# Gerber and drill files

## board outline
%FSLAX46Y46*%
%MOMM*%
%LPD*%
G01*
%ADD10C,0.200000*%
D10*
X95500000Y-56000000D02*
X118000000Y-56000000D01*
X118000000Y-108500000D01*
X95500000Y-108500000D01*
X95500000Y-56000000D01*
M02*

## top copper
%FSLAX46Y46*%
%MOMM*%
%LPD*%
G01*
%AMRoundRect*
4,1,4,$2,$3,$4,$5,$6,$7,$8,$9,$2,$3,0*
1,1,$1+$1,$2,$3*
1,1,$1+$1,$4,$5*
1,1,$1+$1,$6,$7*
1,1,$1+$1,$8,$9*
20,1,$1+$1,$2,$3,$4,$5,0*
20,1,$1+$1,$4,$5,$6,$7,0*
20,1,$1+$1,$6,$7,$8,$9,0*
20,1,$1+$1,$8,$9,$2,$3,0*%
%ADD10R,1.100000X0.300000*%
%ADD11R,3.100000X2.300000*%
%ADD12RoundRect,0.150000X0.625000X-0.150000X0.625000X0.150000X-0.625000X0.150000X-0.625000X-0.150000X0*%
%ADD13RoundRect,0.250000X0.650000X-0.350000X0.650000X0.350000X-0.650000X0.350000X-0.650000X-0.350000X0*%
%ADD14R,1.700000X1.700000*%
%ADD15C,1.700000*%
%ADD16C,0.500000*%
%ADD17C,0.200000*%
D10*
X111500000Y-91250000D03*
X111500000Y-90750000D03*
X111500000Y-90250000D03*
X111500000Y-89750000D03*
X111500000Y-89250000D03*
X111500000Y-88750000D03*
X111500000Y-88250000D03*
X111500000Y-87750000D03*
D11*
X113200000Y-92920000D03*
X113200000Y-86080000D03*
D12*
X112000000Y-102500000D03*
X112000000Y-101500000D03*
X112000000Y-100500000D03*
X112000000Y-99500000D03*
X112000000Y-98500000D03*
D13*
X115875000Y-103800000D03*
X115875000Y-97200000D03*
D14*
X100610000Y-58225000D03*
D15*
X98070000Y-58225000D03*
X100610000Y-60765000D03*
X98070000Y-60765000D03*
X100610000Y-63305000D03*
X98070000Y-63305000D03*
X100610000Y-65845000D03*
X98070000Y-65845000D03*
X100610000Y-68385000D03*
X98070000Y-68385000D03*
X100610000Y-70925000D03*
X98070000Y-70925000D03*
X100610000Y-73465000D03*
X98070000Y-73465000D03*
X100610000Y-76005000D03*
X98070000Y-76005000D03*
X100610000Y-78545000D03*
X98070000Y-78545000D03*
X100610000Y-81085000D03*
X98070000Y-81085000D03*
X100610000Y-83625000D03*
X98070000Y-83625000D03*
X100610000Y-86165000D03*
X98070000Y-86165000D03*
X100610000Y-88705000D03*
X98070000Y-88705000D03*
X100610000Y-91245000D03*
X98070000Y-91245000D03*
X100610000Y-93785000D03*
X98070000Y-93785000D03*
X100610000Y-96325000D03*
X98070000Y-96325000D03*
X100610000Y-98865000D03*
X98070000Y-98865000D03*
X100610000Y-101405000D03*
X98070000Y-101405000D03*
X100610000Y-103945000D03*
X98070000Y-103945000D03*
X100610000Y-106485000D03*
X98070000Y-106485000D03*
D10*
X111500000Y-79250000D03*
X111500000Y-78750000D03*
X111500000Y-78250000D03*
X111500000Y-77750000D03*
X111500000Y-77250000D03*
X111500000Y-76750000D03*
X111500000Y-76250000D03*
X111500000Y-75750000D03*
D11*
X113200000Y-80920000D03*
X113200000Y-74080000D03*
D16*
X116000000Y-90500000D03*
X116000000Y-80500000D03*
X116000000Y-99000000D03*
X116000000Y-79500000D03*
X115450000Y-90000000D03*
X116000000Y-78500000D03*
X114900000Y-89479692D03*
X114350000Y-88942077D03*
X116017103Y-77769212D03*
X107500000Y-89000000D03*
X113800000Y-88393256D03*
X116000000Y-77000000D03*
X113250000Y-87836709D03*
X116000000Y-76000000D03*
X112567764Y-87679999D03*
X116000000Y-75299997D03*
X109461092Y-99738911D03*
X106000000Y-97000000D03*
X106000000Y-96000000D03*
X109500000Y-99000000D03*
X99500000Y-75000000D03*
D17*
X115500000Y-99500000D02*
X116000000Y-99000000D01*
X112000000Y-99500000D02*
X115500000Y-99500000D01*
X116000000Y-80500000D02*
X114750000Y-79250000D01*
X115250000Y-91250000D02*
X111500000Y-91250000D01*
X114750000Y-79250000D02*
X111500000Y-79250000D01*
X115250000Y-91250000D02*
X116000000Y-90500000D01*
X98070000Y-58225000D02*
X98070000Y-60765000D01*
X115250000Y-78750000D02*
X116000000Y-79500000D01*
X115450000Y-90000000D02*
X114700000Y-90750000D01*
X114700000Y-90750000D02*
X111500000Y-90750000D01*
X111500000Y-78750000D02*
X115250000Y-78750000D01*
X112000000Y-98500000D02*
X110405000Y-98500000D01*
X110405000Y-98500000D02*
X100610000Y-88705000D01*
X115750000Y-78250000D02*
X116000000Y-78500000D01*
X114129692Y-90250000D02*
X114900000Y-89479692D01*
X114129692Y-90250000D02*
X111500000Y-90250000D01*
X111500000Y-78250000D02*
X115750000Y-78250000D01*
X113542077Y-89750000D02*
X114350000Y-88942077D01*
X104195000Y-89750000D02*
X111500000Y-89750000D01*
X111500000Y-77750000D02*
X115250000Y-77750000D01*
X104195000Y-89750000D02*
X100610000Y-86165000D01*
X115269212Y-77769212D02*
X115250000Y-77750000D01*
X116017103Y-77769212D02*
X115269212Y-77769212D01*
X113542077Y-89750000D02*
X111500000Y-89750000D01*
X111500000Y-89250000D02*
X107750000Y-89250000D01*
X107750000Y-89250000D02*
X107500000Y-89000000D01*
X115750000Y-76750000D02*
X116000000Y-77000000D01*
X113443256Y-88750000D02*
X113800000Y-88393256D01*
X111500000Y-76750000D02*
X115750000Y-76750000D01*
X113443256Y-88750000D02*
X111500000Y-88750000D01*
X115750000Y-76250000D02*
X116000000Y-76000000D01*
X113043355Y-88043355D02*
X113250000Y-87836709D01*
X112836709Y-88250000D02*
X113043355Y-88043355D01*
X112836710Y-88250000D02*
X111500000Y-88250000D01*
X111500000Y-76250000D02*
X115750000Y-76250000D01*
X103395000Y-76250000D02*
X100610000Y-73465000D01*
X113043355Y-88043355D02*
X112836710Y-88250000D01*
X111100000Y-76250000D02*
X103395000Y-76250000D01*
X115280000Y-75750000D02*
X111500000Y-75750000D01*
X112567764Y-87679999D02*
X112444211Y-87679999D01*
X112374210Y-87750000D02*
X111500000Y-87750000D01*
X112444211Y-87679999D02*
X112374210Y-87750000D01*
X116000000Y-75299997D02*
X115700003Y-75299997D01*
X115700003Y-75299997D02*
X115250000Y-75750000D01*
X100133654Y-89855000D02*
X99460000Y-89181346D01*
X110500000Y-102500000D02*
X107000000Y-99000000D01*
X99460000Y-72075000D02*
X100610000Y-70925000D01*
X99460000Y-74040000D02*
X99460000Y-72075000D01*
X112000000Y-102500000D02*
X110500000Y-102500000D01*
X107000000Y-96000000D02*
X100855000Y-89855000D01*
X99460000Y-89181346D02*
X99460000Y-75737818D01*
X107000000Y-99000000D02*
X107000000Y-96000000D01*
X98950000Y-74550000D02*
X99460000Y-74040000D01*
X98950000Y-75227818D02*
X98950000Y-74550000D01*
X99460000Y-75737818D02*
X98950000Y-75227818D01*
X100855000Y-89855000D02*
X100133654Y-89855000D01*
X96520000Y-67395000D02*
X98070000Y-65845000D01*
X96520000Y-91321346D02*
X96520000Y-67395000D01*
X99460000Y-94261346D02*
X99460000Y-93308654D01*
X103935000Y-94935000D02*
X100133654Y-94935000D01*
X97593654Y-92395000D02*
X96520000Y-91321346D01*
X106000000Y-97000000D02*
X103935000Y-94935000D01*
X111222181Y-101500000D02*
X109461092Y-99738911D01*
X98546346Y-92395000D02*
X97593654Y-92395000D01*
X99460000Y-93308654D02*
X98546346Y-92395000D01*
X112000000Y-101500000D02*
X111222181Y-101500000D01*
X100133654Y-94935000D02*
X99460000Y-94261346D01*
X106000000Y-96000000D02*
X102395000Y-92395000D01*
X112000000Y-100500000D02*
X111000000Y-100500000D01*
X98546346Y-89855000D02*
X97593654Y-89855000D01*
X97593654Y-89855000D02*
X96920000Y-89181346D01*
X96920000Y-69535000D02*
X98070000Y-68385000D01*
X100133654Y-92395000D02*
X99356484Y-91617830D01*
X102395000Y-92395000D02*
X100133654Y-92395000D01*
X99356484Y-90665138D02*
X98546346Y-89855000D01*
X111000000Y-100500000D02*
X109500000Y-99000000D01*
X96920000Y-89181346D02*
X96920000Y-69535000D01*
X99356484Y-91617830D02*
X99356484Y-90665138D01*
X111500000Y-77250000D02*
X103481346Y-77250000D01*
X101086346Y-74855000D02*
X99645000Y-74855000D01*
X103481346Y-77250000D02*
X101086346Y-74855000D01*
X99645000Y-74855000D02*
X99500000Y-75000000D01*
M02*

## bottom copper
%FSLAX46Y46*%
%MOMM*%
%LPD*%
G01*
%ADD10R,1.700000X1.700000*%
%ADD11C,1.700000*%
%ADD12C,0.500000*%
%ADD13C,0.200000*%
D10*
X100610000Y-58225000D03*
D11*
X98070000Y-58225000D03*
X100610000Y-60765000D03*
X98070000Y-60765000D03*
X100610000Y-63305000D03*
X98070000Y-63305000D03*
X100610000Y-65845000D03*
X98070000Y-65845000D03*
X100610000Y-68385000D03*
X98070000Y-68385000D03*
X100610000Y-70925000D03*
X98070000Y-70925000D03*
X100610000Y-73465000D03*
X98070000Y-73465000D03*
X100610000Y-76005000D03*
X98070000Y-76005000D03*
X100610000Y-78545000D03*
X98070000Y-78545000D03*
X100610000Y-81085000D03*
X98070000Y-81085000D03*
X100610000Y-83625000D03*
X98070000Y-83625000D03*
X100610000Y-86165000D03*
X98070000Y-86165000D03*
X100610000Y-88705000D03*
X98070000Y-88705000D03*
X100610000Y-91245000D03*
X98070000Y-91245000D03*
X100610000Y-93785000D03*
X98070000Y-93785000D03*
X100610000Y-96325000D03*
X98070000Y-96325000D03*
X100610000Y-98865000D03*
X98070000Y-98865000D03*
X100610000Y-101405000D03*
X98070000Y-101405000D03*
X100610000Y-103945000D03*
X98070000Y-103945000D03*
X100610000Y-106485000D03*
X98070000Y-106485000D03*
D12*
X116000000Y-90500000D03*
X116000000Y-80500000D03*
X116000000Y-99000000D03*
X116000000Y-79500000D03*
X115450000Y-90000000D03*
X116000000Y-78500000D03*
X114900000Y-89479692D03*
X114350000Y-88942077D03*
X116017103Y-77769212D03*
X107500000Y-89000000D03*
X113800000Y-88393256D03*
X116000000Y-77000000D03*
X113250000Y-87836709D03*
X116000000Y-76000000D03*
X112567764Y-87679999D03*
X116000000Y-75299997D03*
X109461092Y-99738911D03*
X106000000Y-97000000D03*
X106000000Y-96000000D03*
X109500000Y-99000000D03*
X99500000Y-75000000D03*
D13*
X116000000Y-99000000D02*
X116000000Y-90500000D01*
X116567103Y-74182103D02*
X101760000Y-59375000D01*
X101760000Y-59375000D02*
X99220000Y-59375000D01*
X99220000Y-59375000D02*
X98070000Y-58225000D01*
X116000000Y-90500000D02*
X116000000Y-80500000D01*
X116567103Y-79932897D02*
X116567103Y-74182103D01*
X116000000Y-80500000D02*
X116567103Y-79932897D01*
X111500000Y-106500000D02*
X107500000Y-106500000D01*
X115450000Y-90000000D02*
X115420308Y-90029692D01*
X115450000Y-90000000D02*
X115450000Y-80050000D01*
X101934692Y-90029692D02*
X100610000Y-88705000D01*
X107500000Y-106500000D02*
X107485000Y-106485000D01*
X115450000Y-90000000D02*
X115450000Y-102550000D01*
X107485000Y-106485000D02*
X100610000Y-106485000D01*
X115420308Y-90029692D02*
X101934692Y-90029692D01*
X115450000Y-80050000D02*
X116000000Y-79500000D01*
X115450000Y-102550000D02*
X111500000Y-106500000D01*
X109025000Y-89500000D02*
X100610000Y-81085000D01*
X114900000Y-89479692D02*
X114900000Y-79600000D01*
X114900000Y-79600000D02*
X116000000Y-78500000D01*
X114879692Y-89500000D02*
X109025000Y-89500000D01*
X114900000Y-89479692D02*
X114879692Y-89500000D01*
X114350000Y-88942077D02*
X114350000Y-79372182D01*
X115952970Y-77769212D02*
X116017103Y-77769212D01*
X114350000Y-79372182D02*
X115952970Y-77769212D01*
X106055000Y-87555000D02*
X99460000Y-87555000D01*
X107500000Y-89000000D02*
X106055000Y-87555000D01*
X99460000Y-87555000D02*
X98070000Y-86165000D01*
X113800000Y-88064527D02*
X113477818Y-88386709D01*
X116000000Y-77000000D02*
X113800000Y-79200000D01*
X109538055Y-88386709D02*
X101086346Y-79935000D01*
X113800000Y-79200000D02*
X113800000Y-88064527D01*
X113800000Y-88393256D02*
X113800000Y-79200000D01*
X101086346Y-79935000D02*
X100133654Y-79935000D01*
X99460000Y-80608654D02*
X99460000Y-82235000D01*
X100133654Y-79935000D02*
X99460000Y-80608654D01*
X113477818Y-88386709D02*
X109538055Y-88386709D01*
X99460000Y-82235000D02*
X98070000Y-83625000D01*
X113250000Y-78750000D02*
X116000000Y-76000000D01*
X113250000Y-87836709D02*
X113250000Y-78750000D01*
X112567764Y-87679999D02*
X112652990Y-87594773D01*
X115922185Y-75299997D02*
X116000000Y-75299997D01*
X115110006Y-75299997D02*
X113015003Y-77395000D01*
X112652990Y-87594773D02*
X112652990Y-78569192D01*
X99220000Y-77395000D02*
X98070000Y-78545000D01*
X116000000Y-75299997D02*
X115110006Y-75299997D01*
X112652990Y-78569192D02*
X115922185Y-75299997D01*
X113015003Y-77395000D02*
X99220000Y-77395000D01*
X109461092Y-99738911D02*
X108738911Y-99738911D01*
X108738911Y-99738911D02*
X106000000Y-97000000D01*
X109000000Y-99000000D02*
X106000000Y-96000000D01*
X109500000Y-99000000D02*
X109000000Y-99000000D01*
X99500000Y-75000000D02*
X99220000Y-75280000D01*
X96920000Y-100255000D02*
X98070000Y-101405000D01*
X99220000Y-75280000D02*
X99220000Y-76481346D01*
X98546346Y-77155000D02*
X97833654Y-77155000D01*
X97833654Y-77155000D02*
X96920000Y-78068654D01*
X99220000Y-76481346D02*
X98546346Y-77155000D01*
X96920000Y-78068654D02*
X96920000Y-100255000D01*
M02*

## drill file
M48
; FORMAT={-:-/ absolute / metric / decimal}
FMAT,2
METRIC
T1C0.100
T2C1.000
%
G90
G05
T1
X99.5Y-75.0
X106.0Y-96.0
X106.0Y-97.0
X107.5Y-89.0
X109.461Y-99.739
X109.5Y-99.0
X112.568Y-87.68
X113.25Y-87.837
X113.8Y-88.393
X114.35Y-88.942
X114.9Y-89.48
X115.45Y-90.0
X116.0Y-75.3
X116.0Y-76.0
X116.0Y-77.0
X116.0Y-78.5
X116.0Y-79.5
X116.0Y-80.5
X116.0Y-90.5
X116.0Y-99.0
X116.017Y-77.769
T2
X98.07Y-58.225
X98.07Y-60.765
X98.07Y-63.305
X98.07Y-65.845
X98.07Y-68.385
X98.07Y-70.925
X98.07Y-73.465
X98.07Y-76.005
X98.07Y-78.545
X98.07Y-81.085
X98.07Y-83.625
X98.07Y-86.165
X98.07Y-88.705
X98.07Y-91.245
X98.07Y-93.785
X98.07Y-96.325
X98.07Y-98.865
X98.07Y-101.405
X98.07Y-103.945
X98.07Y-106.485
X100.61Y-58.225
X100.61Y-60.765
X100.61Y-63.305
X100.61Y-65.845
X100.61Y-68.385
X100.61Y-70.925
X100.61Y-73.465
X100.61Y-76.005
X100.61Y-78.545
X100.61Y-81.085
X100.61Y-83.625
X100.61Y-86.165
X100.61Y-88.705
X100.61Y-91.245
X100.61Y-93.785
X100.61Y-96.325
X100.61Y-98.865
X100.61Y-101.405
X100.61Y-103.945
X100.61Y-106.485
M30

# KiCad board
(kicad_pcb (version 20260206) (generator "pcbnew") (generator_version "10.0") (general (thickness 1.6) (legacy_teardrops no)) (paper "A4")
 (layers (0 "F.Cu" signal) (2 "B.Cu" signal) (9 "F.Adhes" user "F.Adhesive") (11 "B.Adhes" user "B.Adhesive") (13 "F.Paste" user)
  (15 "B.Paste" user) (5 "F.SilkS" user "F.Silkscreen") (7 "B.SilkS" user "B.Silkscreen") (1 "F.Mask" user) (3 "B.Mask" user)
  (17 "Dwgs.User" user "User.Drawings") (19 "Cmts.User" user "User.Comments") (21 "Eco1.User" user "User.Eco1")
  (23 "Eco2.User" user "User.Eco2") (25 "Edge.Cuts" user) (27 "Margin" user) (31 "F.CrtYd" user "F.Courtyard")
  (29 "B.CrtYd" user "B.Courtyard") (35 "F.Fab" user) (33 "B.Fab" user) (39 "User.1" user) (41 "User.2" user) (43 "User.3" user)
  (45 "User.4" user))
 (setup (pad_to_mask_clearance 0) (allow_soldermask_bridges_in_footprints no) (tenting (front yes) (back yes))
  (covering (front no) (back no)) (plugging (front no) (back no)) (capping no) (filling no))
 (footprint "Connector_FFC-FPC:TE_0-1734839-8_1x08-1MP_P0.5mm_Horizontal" (layer "F.Cu") (at 112.85 89.5 90)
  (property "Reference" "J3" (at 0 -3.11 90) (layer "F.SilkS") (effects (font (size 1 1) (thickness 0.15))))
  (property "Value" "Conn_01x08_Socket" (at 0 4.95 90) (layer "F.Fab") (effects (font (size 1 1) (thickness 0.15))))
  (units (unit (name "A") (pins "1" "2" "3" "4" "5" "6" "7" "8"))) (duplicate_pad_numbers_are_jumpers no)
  (pad "1" smd rect (at -1.75 -1.35 90) (size 0.3 1.1) (layers "F.Cu" "F.Mask" "F.Paste") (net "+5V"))
  (pad "2" smd rect (at -1.25 -1.35 90) (size 0.3 1.1) (layers "F.Cu" "F.Mask" "F.Paste") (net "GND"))
  (pad "3" smd rect (at -0.75 -1.35 90) (size 0.3 1.1) (layers "F.Cu" "F.Mask" "F.Paste") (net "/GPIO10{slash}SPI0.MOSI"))
  (pad "4" smd rect (at -0.25 -1.35 90) (size 0.3 1.1) (layers "F.Cu" "F.Mask" "F.Paste") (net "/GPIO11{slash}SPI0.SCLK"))
  (pad "5" smd rect (at 0.25 -1.35 90) (size 0.3 1.1) (layers "F.Cu" "F.Mask" "F.Paste") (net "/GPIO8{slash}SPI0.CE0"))
  (pad "6" smd rect (at 0.75 -1.35 90) (size 0.3 1.1) (layers "F.Cu" "F.Mask" "F.Paste") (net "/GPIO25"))
  (pad "7" smd rect (at 1.25 -1.35 90) (size 0.3 1.1) (layers "F.Cu" "F.Mask" "F.Paste") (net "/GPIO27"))
  (pad "8" smd rect (at 1.75 -1.35 90) (size 0.3 1.1) (layers "F.Cu" "F.Mask" "F.Paste") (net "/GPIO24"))
  (pad "MP" smd rect (at -3.42 0.35 90) (size 2.3 3.1) (layers "F.Cu" "F.Mask" "F.Paste"))
  (pad "MP" smd rect (at 3.42 0.35 90) (size 2.3 3.1) (layers "F.Cu" "F.Mask" "F.Paste")))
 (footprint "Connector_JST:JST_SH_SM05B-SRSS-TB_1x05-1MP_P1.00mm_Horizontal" (layer "F.Cu") (at 114 100.5 90)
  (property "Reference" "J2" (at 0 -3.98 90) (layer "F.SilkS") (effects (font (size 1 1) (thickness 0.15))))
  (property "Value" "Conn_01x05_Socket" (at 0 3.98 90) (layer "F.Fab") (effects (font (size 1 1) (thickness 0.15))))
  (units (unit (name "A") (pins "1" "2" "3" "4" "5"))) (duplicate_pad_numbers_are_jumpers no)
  (pad "1" smd roundrect (at -2 -2 90) (size 0.6 1.55) (layers "F.Cu" "F.Mask" "F.Paste") (roundrect_rratio 0.25) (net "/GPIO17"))
  (pad "2" smd roundrect (at -1 -2 90) (size 0.6 1.55) (layers "F.Cu" "F.Mask" "F.Paste") (roundrect_rratio 0.25) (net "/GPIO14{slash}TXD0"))
  (pad "3" smd roundrect (at 0 -2 90) (size 0.6 1.55) (layers "F.Cu" "F.Mask" "F.Paste") (roundrect_rratio 0.25) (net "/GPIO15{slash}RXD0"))
  (pad "4" smd roundrect (at 1 -2 90) (size 0.6 1.55) (layers "F.Cu" "F.Mask" "F.Paste") (roundrect_rratio 0.25) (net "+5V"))
  (pad "5" smd roundrect (at 2 -2 90) (size 0.6 1.55) (layers "F.Cu" "F.Mask" "F.Paste") (roundrect_rratio 0.25) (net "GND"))
  (pad "MP" smd roundrect (at -3.3 1.875 90) (size 1.2 1.8) (layers "F.Cu" "F.Mask" "F.Paste") (roundrect_rratio 0.208333))
  (pad "MP" smd roundrect (at 3.3 1.875 90) (size 1.2 1.8) (layers "F.Cu" "F.Mask" "F.Paste") (roundrect_rratio 0.208333)))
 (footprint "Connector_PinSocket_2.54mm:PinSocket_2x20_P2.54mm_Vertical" (layer "F.Cu") (at 100.61 58.225)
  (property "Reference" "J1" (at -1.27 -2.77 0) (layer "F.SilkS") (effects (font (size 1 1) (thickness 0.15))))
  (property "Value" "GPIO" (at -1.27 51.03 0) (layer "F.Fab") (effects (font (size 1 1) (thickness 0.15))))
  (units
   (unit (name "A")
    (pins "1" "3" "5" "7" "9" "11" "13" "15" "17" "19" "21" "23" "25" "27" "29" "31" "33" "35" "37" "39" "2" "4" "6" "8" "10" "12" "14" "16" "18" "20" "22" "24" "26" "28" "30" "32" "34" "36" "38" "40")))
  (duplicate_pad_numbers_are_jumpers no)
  (pad "1" thru_hole rect (at 0 0) (size 1.7 1.7) (drill 1) (layers "*.Cu" "*.Mask") (remove_unused_layers no) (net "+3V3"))
  (pad "2" thru_hole circle (at -2.54 0) (size 1.7 1.7) (drill 1) (layers "*.Cu" "*.Mask") (remove_unused_layers no) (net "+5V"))
  (pad "3" thru_hole circle (at 0 2.54) (size 1.7 1.7) (drill 1) (layers "*.Cu" "*.Mask") (remove_unused_layers no)
   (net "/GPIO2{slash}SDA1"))
  (pad "4" thru_hole circle (at -2.54 2.54) (size 1.7 1.7) (drill 1) (layers "*.Cu" "*.Mask") (remove_unused_layers no) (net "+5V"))
  (pad "5" thru_hole circle (at 0 5.08) (size 1.7 1.7) (drill 1) (layers "*.Cu" "*.Mask") (remove_unused_layers no)
   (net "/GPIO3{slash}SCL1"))
  (pad "6" thru_hole circle (at -2.54 5.08) (size 1.7 1.7) (drill 1) (layers "*.Cu" "*.Mask") (remove_unused_layers no) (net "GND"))
  (pad "7" thru_hole circle (at 0 7.62) (size 1.7 1.7) (drill 1) (layers "*.Cu" "*.Mask") (remove_unused_layers no)
   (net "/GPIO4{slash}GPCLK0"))
  (pad "8" thru_hole circle (at -2.54 7.62) (size 1.7 1.7) (drill 1) (layers "*.Cu" "*.Mask") (remove_unused_layers no)
   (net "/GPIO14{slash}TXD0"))
  (pad "9" thru_hole circle (at 0 10.16) (size 1.7 1.7) (drill 1) (layers "*.Cu" "*.Mask") (remove_unused_layers no) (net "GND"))
  (pad "10" thru_hole circle (at -2.54 10.16) (size 1.7 1.7) (drill 1) (layers "*.Cu" "*.Mask") (remove_unused_layers no)
   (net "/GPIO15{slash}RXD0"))
  (pad "11" thru_hole circle (at 0 12.7) (size 1.7 1.7) (drill 1) (layers "*.Cu" "*.Mask") (remove_unused_layers no) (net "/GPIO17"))
  (pad "12" thru_hole circle (at -2.54 12.7) (size 1.7 1.7) (drill 1) (layers "*.Cu" "*.Mask") (remove_unused_layers no)
   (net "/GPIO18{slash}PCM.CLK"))
  (pad "13" thru_hole circle (at 0 15.24) (size 1.7 1.7) (drill 1) (layers "*.Cu" "*.Mask") (remove_unused_layers no) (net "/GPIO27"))
  (pad "14" thru_hole circle (at -2.54 15.24) (size 1.7 1.7) (drill 1) (layers "*.Cu" "*.Mask") (remove_unused_layers no) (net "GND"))
  (pad "15" thru_hole circle (at 0 17.78) (size 1.7 1.7) (drill 1) (layers "*.Cu" "*.Mask") (remove_unused_layers no) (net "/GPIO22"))
  (pad "16" thru_hole circle (at -2.54 17.78) (size 1.7 1.7) (drill 1) (layers "*.Cu" "*.Mask") (remove_unused_layers no) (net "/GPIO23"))
  (pad "17" thru_hole circle (at 0 20.32) (size 1.7 1.7) (drill 1) (layers "*.Cu" "*.Mask") (remove_unused_layers no) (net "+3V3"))
  (pad "18" thru_hole circle (at -2.54 20.32) (size 1.7 1.7) (drill 1) (layers "*.Cu" "*.Mask") (remove_unused_layers no) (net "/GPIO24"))
  (pad "19" thru_hole circle (at 0 22.86) (size 1.7 1.7) (drill 1) (layers "*.Cu" "*.Mask") (remove_unused_layers no)
   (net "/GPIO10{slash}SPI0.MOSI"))
  (pad "20" thru_hole circle (at -2.54 22.86) (size 1.7 1.7) (drill 1) (layers "*.Cu" "*.Mask") (remove_unused_layers no) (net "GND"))
  (pad "21" thru_hole circle (at 0 25.4) (size 1.7 1.7) (drill 1) (layers "*.Cu" "*.Mask") (remove_unused_layers no)
   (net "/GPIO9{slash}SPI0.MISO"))
  (pad "22" thru_hole circle (at -2.54 25.4) (size 1.7 1.7) (drill 1) (layers "*.Cu" "*.Mask") (remove_unused_layers no) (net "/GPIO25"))
  (pad "23" thru_hole circle (at 0 27.94) (size 1.7 1.7) (drill 1) (layers "*.Cu" "*.Mask") (remove_unused_layers no)
   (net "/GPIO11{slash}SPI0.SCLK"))
  (pad "24" thru_hole circle (at -2.54 27.94) (size 1.7 1.7) (drill 1) (layers "*.Cu" "*.Mask") (remove_unused_layers no)
   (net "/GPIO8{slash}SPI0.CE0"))
  (pad "25" thru_hole circle (at 0 30.48) (size 1.7 1.7) (drill 1) (layers "*.Cu" "*.Mask") (remove_unused_layers no) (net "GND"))
  (pad "26" thru_hole circle (at -2.54 30.48) (size 1.7 1.7) (drill 1) (layers "*.Cu" "*.Mask") (remove_unused_layers no)
   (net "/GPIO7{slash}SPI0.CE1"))
  (pad "27" thru_hole circle (at 0 33.02) (size 1.7 1.7) (drill 1) (layers "*.Cu" "*.Mask") (remove_unused_layers no) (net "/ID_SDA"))
  (pad "28" thru_hole circle (at -2.54 33.02) (size 1.7 1.7) (drill 1) (layers "*.Cu" "*.Mask") (remove_unused_layers no) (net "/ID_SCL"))
  (pad "29" thru_hole circle (at 0 35.56) (size 1.7 1.7) (drill 1) (layers "*.Cu" "*.Mask") (remove_unused_layers no) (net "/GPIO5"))
  (pad "30" thru_hole circle (at -2.54 35.56) (size 1.7 1.7) (drill 1) (layers "*.Cu" "*.Mask") (remove_unused_layers no) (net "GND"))
  (pad "31" thru_hole circle (at 0 38.1) (size 1.7 1.7) (drill 1) (layers "*.Cu" "*.Mask") (remove_unused_layers no) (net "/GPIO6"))
  (pad "32" thru_hole circle (at -2.54 38.1) (size 1.7 1.7) (drill 1) (layers "*.Cu" "*.Mask") (remove_unused_layers no)
   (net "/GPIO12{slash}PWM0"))
  (pad "33" thru_hole circle (at 0 40.64) (size 1.7 1.7) (drill 1) (layers "*.Cu" "*.Mask") (remove_unused_layers no)
   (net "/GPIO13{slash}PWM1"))
  (pad "34" thru_hole circle (at -2.54 40.64) (size 1.7 1.7) (drill 1) (layers "*.Cu" "*.Mask") (remove_unused_layers no) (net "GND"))
  (pad "35" thru_hole circle (at 0 43.18) (size 1.7 1.7) (drill 1) (layers "*.Cu" "*.Mask") (remove_unused_layers no)
   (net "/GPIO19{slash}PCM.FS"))
  (pad "36" thru_hole circle (at -2.54 43.18) (size 1.7 1.7) (drill 1) (layers "*.Cu" "*.Mask") (remove_unused_layers no) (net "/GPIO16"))
  (pad "37" thru_hole circle (at 0 45.72) (size 1.7 1.7) (drill 1) (layers "*.Cu" "*.Mask") (remove_unused_layers no) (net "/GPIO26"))
  (pad "38" thru_hole circle (at -2.54 45.72) (size 1.7 1.7) (drill 1) (layers "*.Cu" "*.Mask") (remove_unused_layers no)
   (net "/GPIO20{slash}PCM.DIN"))
  (pad "39" thru_hole circle (at 0 48.26) (size 1.7 1.7) (drill 1) (layers "*.Cu" "*.Mask") (remove_unused_layers no) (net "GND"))
  (pad "40" thru_hole circle (at -2.54 48.26) (size 1.7 1.7) (drill 1) (layers "*.Cu" "*.Mask") (remove_unused_layers no)
   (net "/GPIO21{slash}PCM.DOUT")))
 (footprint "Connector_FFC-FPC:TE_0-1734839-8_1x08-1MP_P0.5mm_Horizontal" (layer "F.Cu") (at 112.85 77.5 90)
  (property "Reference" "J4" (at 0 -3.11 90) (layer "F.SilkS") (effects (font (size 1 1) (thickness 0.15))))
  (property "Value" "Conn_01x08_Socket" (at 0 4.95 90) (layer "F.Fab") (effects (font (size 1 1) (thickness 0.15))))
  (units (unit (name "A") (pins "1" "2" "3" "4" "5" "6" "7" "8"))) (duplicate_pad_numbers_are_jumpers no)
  (pad "1" smd rect (at -1.75 -1.35 90) (size 0.3 1.1) (layers "F.Cu" "F.Mask" "F.Paste") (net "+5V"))
  (pad "2" smd rect (at -1.25 -1.35 90) (size 0.3 1.1) (layers "F.Cu" "F.Mask" "F.Paste") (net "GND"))
  (pad "3" smd rect (at -0.75 -1.35 90) (size 0.3 1.1) (layers "F.Cu" "F.Mask" "F.Paste") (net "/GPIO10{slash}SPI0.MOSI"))
  (pad "4" smd rect (at -0.25 -1.35 90) (size 0.3 1.1) (layers "F.Cu" "F.Mask" "F.Paste") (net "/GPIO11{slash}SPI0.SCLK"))
  (pad "5" smd rect (at 0.25 -1.35 90) (size 0.3 1.1) (layers "F.Cu" "F.Mask" "F.Paste") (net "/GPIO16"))
  (pad "6" smd rect (at 0.75 -1.35 90) (size 0.3 1.1) (layers "F.Cu" "F.Mask" "F.Paste") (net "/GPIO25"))
  (pad "7" smd rect (at 1.25 -1.35 90) (size 0.3 1.1) (layers "F.Cu" "F.Mask" "F.Paste") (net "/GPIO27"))
  (pad "8" smd rect (at 1.75 -1.35 90) (size 0.3 1.1) (layers "F.Cu" "F.Mask" "F.Paste") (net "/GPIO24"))
  (pad "MP" smd rect (at -3.42 0.35 90) (size 2.3 3.1) (layers "F.Cu" "F.Mask" "F.Paste"))
  (pad "MP" smd rect (at 3.42 0.35 90) (size 2.3 3.1) (layers "F.Cu" "F.Mask" "F.Paste")))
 (gr_rect (start 95.5 56) (end 118 108.5) (stroke (width 0.2) (type solid)) (fill no) (layer "Edge.Cuts"))
 (segment (start 115.5 99.5) (end 116 99) (width 0.2) (layer "F.Cu") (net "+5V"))
 (segment (start 112 99.5) (end 115.5 99.5) (width 0.2) (layer "F.Cu") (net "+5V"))
 (segment (start 116 80.5) (end 114.75 79.25) (width 0.2) (layer "F.Cu") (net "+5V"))
 (segment (start 115.25 91.25) (end 111.5 91.25) (width 0.2) (layer "F.Cu") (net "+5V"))
 (segment (start 114.75 79.25) (end 111.5 79.25) (width 0.2) (layer "F.Cu") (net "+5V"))
 (segment (start 115.25 91.25) (end 116 90.5) (width 0.2) (layer "F.Cu") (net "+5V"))
 (segment (start 98.07 58.225) (end 98.07 60.765) (width 0.2) (layer "F.Cu") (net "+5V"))
 (via micro (at 116 90.5) (size 0.5) (drill 0.1) (layers "F.Cu" "B.Cu") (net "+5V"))
 (via micro (at 116 80.5) (size 0.5) (drill 0.1) (layers "F.Cu" "B.Cu") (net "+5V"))
 (via micro (at 116 99) (size 0.5) (drill 0.1) (layers "F.Cu" "B.Cu") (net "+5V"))
 (segment (start 116 99) (end 116 90.5) (width 0.2) (layer "B.Cu") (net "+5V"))
 (segment (start 116.567103 74.182103) (end 101.76 59.375) (width 0.2) (layer "B.Cu") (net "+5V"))
 (segment (start 101.76 59.375) (end 99.22 59.375) (width 0.2) (layer "B.Cu") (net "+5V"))
 (segment (start 99.22 59.375) (end 98.07 58.225) (width 0.2) (layer "B.Cu") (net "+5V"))
 (segment (start 116 90.5) (end 116 80.5) (width 0.2) (layer "B.Cu") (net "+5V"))
 (segment (start 116.567103 79.932897) (end 116.567103 74.182103) (width 0.2) (layer "B.Cu") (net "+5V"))
 (segment (start 116 80.5) (end 116.567103 79.932897) (width 0.2) (layer "B.Cu") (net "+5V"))
 (segment (start 115.25 78.75) (end 116 79.5) (width 0.2) (layer "F.Cu") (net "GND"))
 (segment (start 115.45 90) (end 114.7 90.75) (width 0.2) (layer "F.Cu") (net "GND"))
 (segment (start 114.7 90.75) (end 111.5 90.75) (width 0.2) (layer "F.Cu") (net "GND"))
 (segment (start 111.5 78.75) (end 115.25 78.75) (width 0.2) (layer "F.Cu") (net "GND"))
 (segment (start 112 98.5) (end 110.405 98.5) (width 0.2) (layer "F.Cu") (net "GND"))
 (segment (start 110.405 98.5) (end 100.61 88.705) (width 0.2) (layer "F.Cu") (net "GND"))
 (via micro (at 116 79.5) (size 0.5) (drill 0.1) (layers "F.Cu" "B.Cu") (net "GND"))
 (via micro (at 115.45 90) (size 0.5) (drill 0.1) (layers "F.Cu" "B.Cu") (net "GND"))
 (segment (start 111.5 106.5) (end 107.5 106.5) (width 0.2) (layer "B.Cu") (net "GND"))
 (segment (start 115.45 90) (end 115.420308 90.029692) (width 0.2) (layer "B.Cu") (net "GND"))
 (segment (start 115.45 90) (end 115.45 80.05) (width 0.2) (layer "B.Cu") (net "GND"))
 (segment (start 101.934692 90.029692) (end 100.61 88.705) (width 0.2) (layer "B.Cu") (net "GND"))
 (segment (start 107.5 106.5) (end 107.485 106.485) (width 0.2) (layer "B.Cu") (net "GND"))
 (segment (start 115.45 90) (end 115.45 102.55) (width 0.2) (layer "B.Cu") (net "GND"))
 (segment (start 107.485 106.485) (end 100.61 106.485) (width 0.2) (layer "B.Cu") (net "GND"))
 (segment (start 115.420308 90.029692) (end 101.934692 90.029692) (width 0.2) (layer "B.Cu") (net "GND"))
 (segment (start 115.45 80.05) (end 116 79.5) (width 0.2) (layer "B.Cu") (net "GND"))
 (segment (start 115.45 102.55) (end 111.5 106.5) (width 0.2) (layer "B.Cu") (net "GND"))
 (segment (start 115.75 78.25) (end 116 78.5) (width 0.2) (layer "F.Cu") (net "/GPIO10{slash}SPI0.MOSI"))
 (segment (start 114.129692 90.25) (end 114.9 89.479692) (width 0.2) (layer "F.Cu") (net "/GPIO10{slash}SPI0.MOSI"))
 (segment (start 114.129692 90.25) (end 111.5 90.25) (width 0.2) (layer "F.Cu") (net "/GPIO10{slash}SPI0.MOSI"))
 (segment (start 111.5 78.25) (end 115.75 78.25) (width 0.2) (layer "F.Cu") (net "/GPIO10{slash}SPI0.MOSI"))
 (via micro (at 116 78.5) (size 0.5) (drill 0.1) (layers "F.Cu" "B.Cu") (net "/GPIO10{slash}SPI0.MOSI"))
 (via micro (at 114.9 89.479692) (size 0.5) (drill 0.1) (layers "F.Cu" "B.Cu") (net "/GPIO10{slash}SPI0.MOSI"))
 (segment (start 109.025 89.5) (end 100.61 81.085) (width 0.2) (layer "B.Cu") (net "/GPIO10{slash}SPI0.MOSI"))
 (segment (start 114.9 89.479692) (end 114.9 79.6) (width 0.2) (layer "B.Cu") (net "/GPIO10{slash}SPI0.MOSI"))
 (segment (start 114.9 79.6) (end 116 78.5) (width 0.2) (layer "B.Cu") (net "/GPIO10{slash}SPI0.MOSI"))
 (segment (start 114.879692 89.5) (end 109.025 89.5) (width 0.2) (layer "B.Cu") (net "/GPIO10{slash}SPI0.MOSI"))
 (segment (start 114.9 89.479692) (end 114.879692 89.5) (width 0.2) (layer "B.Cu") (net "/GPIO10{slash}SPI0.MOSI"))
 (segment (start 113.542077 89.75) (end 114.35 88.942077) (width 0.2) (layer "F.Cu") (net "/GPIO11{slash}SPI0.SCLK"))
 (segment (start 104.195 89.75) (end 111.5 89.75) (width 0.2) (layer "F.Cu") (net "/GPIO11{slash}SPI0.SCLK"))
 (segment (start 111.5 77.75) (end 115.25 77.75) (width 0.2) (layer "F.Cu") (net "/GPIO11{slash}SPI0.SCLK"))
 (segment (start 104.195 89.75) (end 100.61 86.165) (width 0.2) (layer "F.Cu") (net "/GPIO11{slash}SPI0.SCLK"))
 (segment (start 115.269212 77.769212) (end 115.25 77.75) (width 0.2) (layer "F.Cu") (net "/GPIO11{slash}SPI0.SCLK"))
 (segment (start 116.017103 77.769212) (end 115.269212 77.769212) (width 0.2) (layer "F.Cu") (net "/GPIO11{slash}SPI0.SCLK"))
 (segment (start 113.542077 89.75) (end 111.5 89.75) (width 0.2) (layer "F.Cu") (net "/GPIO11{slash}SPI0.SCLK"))
 (via micro (at 114.35 88.942077) (size 0.5) (drill 0.1) (layers "F.Cu" "B.Cu") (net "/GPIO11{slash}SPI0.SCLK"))
 (via micro (at 116.017103 77.769212) (size 0.5) (drill 0.1) (layers "F.Cu" "B.Cu") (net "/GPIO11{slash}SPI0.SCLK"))
 (segment (start 114.35 88.942077) (end 114.35 79.372182) (width 0.2) (layer "B.Cu") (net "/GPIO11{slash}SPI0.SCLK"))
 (segment (start 115.95297 77.769212) (end 116.017103 77.769212) (width 0.2) (layer "B.Cu") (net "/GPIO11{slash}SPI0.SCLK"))
 (segment (start 114.35 79.372182) (end 115.95297 77.769212) (width 0.2) (layer "B.Cu") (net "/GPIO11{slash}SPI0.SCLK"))
 (segment (start 111.5 89.25) (end 107.75 89.25) (width 0.2) (layer "F.Cu") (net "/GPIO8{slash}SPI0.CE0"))
 (segment (start 107.75 89.25) (end 107.5 89) (width 0.2) (layer "F.Cu") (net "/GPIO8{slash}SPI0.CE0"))
 (via micro (at 107.5 89) (size 0.5) (drill 0.1) (layers "F.Cu" "B.Cu") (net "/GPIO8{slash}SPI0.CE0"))
 (segment (start 106.055 87.555) (end 99.46 87.555) (width 0.2) (layer "B.Cu") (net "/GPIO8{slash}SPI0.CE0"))
 (segment (start 107.5 89) (end 106.055 87.555) (width 0.2) (layer "B.Cu") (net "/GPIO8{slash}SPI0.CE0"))
 (segment (start 99.46 87.555) (end 98.07 86.165) (width 0.2) (layer "B.Cu") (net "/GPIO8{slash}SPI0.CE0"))
 (segment (start 115.75 76.75) (end 116 77) (width 0.2) (layer "F.Cu") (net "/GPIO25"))
 (segment (start 113.443256 88.75) (end 113.8 88.393256) (width 0.2) (layer "F.Cu") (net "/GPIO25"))
 (segment (start 111.5 76.75) (end 115.75 76.75) (width 0.2) (layer "F.Cu") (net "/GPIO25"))
 (segment (start 113.443256 88.75) (end 111.5 88.75) (width 0.2) (layer "F.Cu") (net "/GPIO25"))
 (via micro (at 113.8 88.393256) (size 0.5) (drill 0.1) (layers "F.Cu" "B.Cu") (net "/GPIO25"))
 (via micro (at 116 77) (size 0.5) (drill 0.1) (layers "F.Cu" "B.Cu") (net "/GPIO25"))
 (segment (start 113.8 88.064527) (end 113.477818 88.386709) (width 0.2) (layer "B.Cu") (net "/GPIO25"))
 (segment (start 116 77) (end 113.8 79.2) (width 0.2) (layer "B.Cu") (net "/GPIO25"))
 (segment (start 109.538055 88.386709) (end 101.086346 79.935) (width 0.2) (layer "B.Cu") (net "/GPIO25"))
 (segment (start 113.8 79.2) (end 113.8 88.064527) (width 0.2) (layer "B.Cu") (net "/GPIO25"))
 (segment (start 113.8 88.393256) (end 113.8 79.2) (width 0.2) (layer "B.Cu") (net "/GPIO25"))
 (segment (start 101.086346 79.935) (end 100.133654 79.935) (width 0.2) (layer "B.Cu") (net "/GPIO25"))
 (segment (start 99.46 80.608654) (end 99.46 82.235) (width 0.2) (layer "B.Cu") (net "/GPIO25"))
 (segment (start 100.133654 79.935) (end 99.46 80.608654) (width 0.2) (layer "B.Cu") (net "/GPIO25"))
 (segment (start 113.477818 88.386709) (end 109.538055 88.386709) (width 0.2) (layer "B.Cu") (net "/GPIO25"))
 (segment (start 99.46 82.235) (end 98.07 83.625) (width 0.2) (layer "B.Cu") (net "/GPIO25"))
 (segment (start 115.75 76.25) (end 116 76) (width 0.2) (layer "F.Cu") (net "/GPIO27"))
 (segment (start 113.043355 88.043355) (end 113.25 87.836709) (width 0.2) (layer "F.Cu") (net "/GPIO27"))
 (segment (start 112.836709 88.25) (end 113.043355 88.043355) (width 0.2) (layer "F.Cu") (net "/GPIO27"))
 (segment (start 112.83671 88.25) (end 111.5 88.25) (width 0.2) (layer "F.Cu") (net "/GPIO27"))
 (segment (start 111.5 76.25) (end 115.75 76.25) (width 0.2) (layer "F.Cu") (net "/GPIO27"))
 (segment (start 103.395 76.25) (end 100.61 73.465) (width 0.2) (layer "F.Cu") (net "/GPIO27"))
 (segment (start 113.043355 88.043355) (end 112.83671 88.25) (width 0.2) (layer "F.Cu") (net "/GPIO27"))
 (segment (start 111.1 76.25) (end 103.395 76.25) (width 0.2) (layer "F.Cu") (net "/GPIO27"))
 (via micro (at 113.25 87.836709) (size 0.5) (drill 0.1) (layers "F.Cu" "B.Cu") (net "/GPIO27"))
 (via micro (at 116 76) (size 0.5) (drill 0.1) (layers "F.Cu" "B.Cu") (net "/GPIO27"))
 (segment (start 113.25 78.75) (end 116 76) (width 0.2) (layer "B.Cu") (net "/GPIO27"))
 (segment (start 113.25 87.836709) (end 113.25 78.75) (width 0.2) (layer "B.Cu") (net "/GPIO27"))
 (segment (start 115.28 75.75) (end 111.5 75.75) (width 0.2) (layer "F.Cu") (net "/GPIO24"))
 (segment (start 112.567764 87.679999) (end 112.444211 87.679999) (width 0.2) (layer "F.Cu") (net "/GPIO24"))
 (segment (start 112.37421 87.75) (end 111.5 87.75) (width 0.2) (layer "F.Cu") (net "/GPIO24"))
 (segment (start 112.444211 87.679999) (end 112.37421 87.75) (width 0.2) (layer "F.Cu") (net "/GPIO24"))
 (segment (start 116 75.299997) (end 115.700003 75.299997) (width 0.2) (layer "F.Cu") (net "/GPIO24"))
 (segment (start 115.700003 75.299997) (end 115.25 75.75) (width 0.2) (layer "F.Cu") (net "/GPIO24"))
 (via micro (at 112.567764 87.679999) (size 0.5) (drill 0.1) (layers "F.Cu" "B.Cu") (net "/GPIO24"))
 (via micro (at 116 75.299997) (size 0.5) (drill 0.1) (layers "F.Cu" "B.Cu") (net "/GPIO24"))
 (segment (start 112.567764 87.679999) (end 112.65299 87.594773) (width 0.2) (layer "B.Cu") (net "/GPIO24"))
 (segment (start 115.922185 75.299997) (end 116 75.299997) (width 0.2) (layer "B.Cu") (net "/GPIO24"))
 (segment (start 115.110006 75.299997) (end 113.015003 77.395) (width 0.2) (layer "B.Cu") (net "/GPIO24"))
 (segment (start 112.65299 87.594773) (end 112.65299 78.569192) (width 0.2) (layer "B.Cu") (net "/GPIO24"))
 (segment (start 99.22 77.395) (end 98.07 78.545) (width 0.2) (layer "B.Cu") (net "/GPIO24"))
 (segment (start 116 75.299997) (end 115.110006 75.299997) (width 0.2) (layer "B.Cu") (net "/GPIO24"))
 (segment (start 112.65299 78.569192) (end 115.922185 75.299997) (width 0.2) (layer "B.Cu") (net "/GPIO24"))
 (segment (start 113.015003 77.395) (end 99.22 77.395) (width 0.2) (layer "B.Cu") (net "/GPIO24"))
 (segment (start 100.133654 89.855) (end 99.46 89.181346) (width 0.2) (layer "F.Cu") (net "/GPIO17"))
 (segment (start 110.5 102.5) (end 107 99) (width 0.2) (layer "F.Cu") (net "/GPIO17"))
 (segment (start 99.46 72.075) (end 100.61 70.925) (width 0.2) (layer "F.Cu") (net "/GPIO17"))
 (segment (start 99.46 74.04) (end 99.46 72.075) (width 0.2) (layer "F.Cu") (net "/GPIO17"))
 (segment (start 112 102.5) (end 110.5 102.5) (width 0.2) (layer "F.Cu") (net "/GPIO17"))
 (segment (start 107 96) (end 100.855 89.855) (width 0.2) (layer "F.Cu") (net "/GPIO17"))
 (segment (start 99.46 89.181346) (end 99.46 75.737818) (width 0.2) (layer "F.Cu") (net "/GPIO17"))
 (segment (start 107 99) (end 107 96) (width 0.2) (layer "F.Cu") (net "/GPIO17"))
 (segment (start 98.95 74.55) (end 99.46 74.04) (width 0.2) (layer "F.Cu") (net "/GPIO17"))
 (segment (start 98.95 75.227818) (end 98.95 74.55) (width 0.2) (layer "F.Cu") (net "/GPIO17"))
 (segment (start 99.46 75.737818) (end 98.95 75.227818) (width 0.2) (layer "F.Cu") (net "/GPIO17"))
 (segment (start 100.855 89.855) (end 100.133654 89.855) (width 0.2) (layer "F.Cu") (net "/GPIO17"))
 (segment (start 96.52 67.395) (end 98.07 65.845) (width 0.2) (layer "F.Cu") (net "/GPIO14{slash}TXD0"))
 (segment (start 96.52 91.321346) (end 96.52 67.395) (width 0.2) (layer "F.Cu") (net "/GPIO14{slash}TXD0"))
 (segment (start 99.46 94.261346) (end 99.46 93.308654) (width 0.2) (layer "F.Cu") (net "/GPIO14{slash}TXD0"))
 (segment (start 103.935 94.935) (end 100.133654 94.935) (width 0.2) (layer "F.Cu") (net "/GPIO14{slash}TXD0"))
 (segment (start 97.593654 92.395) (end 96.52 91.321346) (width 0.2) (layer "F.Cu") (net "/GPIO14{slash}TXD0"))
 (segment (start 106 97) (end 103.935 94.935) (width 0.2) (layer "F.Cu") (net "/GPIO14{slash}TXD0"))
 (segment (start 111.222181 101.5) (end 109.461092 99.738911) (width 0.2) (layer "F.Cu") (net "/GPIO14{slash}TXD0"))
 (segment (start 98.546346 92.395) (end 97.593654 92.395) (width 0.2) (layer "F.Cu") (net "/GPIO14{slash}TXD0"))
 (segment (start 99.46 93.308654) (end 98.546346 92.395) (width 0.2) (layer "F.Cu") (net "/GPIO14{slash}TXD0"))
 (segment (start 112 101.5) (end 111.222181 101.5) (width 0.2) (layer "F.Cu") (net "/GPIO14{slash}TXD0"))
 (segment (start 100.133654 94.935) (end 99.46 94.261346) (width 0.2) (layer "F.Cu") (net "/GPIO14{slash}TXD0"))
 (via micro (at 109.461092 99.738911) (size 0.5) (drill 0.1) (layers "F.Cu" "B.Cu") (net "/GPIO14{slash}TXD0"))
 (via micro (at 106 97) (size 0.5) (drill 0.1) (layers "F.Cu" "B.Cu") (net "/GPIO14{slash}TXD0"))
 (segment (start 109.461092 99.738911) (end 108.738911 99.738911) (width 0.2) (layer "B.Cu") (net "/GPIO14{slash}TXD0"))
 (segment (start 108.738911 99.738911) (end 106 97) (width 0.2) (layer "B.Cu") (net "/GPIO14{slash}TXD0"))
 (segment (start 106 96) (end 102.395 92.395) (width 0.2) (layer "F.Cu") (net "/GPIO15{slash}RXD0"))
 (segment (start 112 100.5) (end 111 100.5) (width 0.2) (layer "F.Cu") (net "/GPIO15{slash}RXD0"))
 (segment (start 98.546346 89.855) (end 97.593654 89.855) (width 0.2) (layer "F.Cu") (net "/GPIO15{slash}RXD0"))
 (segment (start 97.593654 89.855) (end 96.92 89.181346) (width 0.2) (layer "F.Cu") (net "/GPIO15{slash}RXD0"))
 (segment (start 96.92 69.535) (end 98.07 68.385) (width 0.2) (layer "F.Cu") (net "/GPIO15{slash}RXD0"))
 (segment (start 100.133654 92.395) (end 99.356484 91.61783) (width 0.2) (layer "F.Cu") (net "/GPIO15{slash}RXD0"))
 (segment (start 102.395 92.395) (end 100.133654 92.395) (width 0.2) (layer "F.Cu") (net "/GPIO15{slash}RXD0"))
 (segment (start 99.356484 90.665138) (end 98.546346 89.855) (width 0.2) (layer "F.Cu") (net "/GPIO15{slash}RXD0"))
 (segment (start 111 100.5) (end 109.5 99) (width 0.2) (layer "F.Cu") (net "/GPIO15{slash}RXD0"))
 (segment (start 96.92 89.181346) (end 96.92 69.535) (width 0.2) (layer "F.Cu") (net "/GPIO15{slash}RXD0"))
 (segment (start 99.356484 91.61783) (end 99.356484 90.665138) (width 0.2) (layer "F.Cu") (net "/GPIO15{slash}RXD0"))
 (via micro (at 106 96) (size 0.5) (drill 0.1) (layers "F.Cu" "B.Cu") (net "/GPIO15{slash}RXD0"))
 (via micro (at 109.5 99) (size 0.5) (drill 0.1) (layers "F.Cu" "B.Cu") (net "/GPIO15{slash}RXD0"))
 (segment (start 109 99) (end 106 96) (width 0.2) (layer "B.Cu") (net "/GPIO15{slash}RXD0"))
 (segment (start 109.5 99) (end 109 99) (width 0.2) (layer "B.Cu") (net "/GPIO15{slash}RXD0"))
 (segment (start 111.5 77.25) (end 103.481346 77.25) (width 0.2) (layer "F.Cu") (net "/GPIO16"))
 (segment (start 101.086346 74.855) (end 99.645 74.855) (width 0.2) (layer "F.Cu") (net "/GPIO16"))
 (segment (start 103.481346 77.25) (end 101.086346 74.855) (width 0.2) (layer "F.Cu") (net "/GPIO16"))
 (segment (start 99.645 74.855) (end 99.5 75) (width 0.2) (layer "F.Cu") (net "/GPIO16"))
 (via micro (at 99.5 75) (size 0.5) (drill 0.1) (layers "F.Cu" "B.Cu") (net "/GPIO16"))
 (segment (start 99.5 75) (end 99.22 75.28) (width 0.2) (layer "B.Cu") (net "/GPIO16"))
 (segment (start 96.92 100.255) (end 98.07 101.405) (width 0.2) (layer "B.Cu") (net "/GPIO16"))
 (segment (start 99.22 75.28) (end 99.22 76.481346) (width 0.2) (layer "B.Cu") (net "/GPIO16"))
 (segment (start 98.546346 77.155) (end 97.833654 77.155) (width 0.2) (layer "B.Cu") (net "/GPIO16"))
 (segment (start 97.833654 77.155) (end 96.92 78.068654) (width 0.2) (layer "B.Cu") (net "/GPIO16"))
 (segment (start 99.22 76.481346) (end 98.546346 77.155) (width 0.2) (layer "B.Cu") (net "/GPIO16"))
 (segment (start 96.92 78.068654) (end 96.92 100.255) (width 0.2) (layer "B.Cu") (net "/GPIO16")))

